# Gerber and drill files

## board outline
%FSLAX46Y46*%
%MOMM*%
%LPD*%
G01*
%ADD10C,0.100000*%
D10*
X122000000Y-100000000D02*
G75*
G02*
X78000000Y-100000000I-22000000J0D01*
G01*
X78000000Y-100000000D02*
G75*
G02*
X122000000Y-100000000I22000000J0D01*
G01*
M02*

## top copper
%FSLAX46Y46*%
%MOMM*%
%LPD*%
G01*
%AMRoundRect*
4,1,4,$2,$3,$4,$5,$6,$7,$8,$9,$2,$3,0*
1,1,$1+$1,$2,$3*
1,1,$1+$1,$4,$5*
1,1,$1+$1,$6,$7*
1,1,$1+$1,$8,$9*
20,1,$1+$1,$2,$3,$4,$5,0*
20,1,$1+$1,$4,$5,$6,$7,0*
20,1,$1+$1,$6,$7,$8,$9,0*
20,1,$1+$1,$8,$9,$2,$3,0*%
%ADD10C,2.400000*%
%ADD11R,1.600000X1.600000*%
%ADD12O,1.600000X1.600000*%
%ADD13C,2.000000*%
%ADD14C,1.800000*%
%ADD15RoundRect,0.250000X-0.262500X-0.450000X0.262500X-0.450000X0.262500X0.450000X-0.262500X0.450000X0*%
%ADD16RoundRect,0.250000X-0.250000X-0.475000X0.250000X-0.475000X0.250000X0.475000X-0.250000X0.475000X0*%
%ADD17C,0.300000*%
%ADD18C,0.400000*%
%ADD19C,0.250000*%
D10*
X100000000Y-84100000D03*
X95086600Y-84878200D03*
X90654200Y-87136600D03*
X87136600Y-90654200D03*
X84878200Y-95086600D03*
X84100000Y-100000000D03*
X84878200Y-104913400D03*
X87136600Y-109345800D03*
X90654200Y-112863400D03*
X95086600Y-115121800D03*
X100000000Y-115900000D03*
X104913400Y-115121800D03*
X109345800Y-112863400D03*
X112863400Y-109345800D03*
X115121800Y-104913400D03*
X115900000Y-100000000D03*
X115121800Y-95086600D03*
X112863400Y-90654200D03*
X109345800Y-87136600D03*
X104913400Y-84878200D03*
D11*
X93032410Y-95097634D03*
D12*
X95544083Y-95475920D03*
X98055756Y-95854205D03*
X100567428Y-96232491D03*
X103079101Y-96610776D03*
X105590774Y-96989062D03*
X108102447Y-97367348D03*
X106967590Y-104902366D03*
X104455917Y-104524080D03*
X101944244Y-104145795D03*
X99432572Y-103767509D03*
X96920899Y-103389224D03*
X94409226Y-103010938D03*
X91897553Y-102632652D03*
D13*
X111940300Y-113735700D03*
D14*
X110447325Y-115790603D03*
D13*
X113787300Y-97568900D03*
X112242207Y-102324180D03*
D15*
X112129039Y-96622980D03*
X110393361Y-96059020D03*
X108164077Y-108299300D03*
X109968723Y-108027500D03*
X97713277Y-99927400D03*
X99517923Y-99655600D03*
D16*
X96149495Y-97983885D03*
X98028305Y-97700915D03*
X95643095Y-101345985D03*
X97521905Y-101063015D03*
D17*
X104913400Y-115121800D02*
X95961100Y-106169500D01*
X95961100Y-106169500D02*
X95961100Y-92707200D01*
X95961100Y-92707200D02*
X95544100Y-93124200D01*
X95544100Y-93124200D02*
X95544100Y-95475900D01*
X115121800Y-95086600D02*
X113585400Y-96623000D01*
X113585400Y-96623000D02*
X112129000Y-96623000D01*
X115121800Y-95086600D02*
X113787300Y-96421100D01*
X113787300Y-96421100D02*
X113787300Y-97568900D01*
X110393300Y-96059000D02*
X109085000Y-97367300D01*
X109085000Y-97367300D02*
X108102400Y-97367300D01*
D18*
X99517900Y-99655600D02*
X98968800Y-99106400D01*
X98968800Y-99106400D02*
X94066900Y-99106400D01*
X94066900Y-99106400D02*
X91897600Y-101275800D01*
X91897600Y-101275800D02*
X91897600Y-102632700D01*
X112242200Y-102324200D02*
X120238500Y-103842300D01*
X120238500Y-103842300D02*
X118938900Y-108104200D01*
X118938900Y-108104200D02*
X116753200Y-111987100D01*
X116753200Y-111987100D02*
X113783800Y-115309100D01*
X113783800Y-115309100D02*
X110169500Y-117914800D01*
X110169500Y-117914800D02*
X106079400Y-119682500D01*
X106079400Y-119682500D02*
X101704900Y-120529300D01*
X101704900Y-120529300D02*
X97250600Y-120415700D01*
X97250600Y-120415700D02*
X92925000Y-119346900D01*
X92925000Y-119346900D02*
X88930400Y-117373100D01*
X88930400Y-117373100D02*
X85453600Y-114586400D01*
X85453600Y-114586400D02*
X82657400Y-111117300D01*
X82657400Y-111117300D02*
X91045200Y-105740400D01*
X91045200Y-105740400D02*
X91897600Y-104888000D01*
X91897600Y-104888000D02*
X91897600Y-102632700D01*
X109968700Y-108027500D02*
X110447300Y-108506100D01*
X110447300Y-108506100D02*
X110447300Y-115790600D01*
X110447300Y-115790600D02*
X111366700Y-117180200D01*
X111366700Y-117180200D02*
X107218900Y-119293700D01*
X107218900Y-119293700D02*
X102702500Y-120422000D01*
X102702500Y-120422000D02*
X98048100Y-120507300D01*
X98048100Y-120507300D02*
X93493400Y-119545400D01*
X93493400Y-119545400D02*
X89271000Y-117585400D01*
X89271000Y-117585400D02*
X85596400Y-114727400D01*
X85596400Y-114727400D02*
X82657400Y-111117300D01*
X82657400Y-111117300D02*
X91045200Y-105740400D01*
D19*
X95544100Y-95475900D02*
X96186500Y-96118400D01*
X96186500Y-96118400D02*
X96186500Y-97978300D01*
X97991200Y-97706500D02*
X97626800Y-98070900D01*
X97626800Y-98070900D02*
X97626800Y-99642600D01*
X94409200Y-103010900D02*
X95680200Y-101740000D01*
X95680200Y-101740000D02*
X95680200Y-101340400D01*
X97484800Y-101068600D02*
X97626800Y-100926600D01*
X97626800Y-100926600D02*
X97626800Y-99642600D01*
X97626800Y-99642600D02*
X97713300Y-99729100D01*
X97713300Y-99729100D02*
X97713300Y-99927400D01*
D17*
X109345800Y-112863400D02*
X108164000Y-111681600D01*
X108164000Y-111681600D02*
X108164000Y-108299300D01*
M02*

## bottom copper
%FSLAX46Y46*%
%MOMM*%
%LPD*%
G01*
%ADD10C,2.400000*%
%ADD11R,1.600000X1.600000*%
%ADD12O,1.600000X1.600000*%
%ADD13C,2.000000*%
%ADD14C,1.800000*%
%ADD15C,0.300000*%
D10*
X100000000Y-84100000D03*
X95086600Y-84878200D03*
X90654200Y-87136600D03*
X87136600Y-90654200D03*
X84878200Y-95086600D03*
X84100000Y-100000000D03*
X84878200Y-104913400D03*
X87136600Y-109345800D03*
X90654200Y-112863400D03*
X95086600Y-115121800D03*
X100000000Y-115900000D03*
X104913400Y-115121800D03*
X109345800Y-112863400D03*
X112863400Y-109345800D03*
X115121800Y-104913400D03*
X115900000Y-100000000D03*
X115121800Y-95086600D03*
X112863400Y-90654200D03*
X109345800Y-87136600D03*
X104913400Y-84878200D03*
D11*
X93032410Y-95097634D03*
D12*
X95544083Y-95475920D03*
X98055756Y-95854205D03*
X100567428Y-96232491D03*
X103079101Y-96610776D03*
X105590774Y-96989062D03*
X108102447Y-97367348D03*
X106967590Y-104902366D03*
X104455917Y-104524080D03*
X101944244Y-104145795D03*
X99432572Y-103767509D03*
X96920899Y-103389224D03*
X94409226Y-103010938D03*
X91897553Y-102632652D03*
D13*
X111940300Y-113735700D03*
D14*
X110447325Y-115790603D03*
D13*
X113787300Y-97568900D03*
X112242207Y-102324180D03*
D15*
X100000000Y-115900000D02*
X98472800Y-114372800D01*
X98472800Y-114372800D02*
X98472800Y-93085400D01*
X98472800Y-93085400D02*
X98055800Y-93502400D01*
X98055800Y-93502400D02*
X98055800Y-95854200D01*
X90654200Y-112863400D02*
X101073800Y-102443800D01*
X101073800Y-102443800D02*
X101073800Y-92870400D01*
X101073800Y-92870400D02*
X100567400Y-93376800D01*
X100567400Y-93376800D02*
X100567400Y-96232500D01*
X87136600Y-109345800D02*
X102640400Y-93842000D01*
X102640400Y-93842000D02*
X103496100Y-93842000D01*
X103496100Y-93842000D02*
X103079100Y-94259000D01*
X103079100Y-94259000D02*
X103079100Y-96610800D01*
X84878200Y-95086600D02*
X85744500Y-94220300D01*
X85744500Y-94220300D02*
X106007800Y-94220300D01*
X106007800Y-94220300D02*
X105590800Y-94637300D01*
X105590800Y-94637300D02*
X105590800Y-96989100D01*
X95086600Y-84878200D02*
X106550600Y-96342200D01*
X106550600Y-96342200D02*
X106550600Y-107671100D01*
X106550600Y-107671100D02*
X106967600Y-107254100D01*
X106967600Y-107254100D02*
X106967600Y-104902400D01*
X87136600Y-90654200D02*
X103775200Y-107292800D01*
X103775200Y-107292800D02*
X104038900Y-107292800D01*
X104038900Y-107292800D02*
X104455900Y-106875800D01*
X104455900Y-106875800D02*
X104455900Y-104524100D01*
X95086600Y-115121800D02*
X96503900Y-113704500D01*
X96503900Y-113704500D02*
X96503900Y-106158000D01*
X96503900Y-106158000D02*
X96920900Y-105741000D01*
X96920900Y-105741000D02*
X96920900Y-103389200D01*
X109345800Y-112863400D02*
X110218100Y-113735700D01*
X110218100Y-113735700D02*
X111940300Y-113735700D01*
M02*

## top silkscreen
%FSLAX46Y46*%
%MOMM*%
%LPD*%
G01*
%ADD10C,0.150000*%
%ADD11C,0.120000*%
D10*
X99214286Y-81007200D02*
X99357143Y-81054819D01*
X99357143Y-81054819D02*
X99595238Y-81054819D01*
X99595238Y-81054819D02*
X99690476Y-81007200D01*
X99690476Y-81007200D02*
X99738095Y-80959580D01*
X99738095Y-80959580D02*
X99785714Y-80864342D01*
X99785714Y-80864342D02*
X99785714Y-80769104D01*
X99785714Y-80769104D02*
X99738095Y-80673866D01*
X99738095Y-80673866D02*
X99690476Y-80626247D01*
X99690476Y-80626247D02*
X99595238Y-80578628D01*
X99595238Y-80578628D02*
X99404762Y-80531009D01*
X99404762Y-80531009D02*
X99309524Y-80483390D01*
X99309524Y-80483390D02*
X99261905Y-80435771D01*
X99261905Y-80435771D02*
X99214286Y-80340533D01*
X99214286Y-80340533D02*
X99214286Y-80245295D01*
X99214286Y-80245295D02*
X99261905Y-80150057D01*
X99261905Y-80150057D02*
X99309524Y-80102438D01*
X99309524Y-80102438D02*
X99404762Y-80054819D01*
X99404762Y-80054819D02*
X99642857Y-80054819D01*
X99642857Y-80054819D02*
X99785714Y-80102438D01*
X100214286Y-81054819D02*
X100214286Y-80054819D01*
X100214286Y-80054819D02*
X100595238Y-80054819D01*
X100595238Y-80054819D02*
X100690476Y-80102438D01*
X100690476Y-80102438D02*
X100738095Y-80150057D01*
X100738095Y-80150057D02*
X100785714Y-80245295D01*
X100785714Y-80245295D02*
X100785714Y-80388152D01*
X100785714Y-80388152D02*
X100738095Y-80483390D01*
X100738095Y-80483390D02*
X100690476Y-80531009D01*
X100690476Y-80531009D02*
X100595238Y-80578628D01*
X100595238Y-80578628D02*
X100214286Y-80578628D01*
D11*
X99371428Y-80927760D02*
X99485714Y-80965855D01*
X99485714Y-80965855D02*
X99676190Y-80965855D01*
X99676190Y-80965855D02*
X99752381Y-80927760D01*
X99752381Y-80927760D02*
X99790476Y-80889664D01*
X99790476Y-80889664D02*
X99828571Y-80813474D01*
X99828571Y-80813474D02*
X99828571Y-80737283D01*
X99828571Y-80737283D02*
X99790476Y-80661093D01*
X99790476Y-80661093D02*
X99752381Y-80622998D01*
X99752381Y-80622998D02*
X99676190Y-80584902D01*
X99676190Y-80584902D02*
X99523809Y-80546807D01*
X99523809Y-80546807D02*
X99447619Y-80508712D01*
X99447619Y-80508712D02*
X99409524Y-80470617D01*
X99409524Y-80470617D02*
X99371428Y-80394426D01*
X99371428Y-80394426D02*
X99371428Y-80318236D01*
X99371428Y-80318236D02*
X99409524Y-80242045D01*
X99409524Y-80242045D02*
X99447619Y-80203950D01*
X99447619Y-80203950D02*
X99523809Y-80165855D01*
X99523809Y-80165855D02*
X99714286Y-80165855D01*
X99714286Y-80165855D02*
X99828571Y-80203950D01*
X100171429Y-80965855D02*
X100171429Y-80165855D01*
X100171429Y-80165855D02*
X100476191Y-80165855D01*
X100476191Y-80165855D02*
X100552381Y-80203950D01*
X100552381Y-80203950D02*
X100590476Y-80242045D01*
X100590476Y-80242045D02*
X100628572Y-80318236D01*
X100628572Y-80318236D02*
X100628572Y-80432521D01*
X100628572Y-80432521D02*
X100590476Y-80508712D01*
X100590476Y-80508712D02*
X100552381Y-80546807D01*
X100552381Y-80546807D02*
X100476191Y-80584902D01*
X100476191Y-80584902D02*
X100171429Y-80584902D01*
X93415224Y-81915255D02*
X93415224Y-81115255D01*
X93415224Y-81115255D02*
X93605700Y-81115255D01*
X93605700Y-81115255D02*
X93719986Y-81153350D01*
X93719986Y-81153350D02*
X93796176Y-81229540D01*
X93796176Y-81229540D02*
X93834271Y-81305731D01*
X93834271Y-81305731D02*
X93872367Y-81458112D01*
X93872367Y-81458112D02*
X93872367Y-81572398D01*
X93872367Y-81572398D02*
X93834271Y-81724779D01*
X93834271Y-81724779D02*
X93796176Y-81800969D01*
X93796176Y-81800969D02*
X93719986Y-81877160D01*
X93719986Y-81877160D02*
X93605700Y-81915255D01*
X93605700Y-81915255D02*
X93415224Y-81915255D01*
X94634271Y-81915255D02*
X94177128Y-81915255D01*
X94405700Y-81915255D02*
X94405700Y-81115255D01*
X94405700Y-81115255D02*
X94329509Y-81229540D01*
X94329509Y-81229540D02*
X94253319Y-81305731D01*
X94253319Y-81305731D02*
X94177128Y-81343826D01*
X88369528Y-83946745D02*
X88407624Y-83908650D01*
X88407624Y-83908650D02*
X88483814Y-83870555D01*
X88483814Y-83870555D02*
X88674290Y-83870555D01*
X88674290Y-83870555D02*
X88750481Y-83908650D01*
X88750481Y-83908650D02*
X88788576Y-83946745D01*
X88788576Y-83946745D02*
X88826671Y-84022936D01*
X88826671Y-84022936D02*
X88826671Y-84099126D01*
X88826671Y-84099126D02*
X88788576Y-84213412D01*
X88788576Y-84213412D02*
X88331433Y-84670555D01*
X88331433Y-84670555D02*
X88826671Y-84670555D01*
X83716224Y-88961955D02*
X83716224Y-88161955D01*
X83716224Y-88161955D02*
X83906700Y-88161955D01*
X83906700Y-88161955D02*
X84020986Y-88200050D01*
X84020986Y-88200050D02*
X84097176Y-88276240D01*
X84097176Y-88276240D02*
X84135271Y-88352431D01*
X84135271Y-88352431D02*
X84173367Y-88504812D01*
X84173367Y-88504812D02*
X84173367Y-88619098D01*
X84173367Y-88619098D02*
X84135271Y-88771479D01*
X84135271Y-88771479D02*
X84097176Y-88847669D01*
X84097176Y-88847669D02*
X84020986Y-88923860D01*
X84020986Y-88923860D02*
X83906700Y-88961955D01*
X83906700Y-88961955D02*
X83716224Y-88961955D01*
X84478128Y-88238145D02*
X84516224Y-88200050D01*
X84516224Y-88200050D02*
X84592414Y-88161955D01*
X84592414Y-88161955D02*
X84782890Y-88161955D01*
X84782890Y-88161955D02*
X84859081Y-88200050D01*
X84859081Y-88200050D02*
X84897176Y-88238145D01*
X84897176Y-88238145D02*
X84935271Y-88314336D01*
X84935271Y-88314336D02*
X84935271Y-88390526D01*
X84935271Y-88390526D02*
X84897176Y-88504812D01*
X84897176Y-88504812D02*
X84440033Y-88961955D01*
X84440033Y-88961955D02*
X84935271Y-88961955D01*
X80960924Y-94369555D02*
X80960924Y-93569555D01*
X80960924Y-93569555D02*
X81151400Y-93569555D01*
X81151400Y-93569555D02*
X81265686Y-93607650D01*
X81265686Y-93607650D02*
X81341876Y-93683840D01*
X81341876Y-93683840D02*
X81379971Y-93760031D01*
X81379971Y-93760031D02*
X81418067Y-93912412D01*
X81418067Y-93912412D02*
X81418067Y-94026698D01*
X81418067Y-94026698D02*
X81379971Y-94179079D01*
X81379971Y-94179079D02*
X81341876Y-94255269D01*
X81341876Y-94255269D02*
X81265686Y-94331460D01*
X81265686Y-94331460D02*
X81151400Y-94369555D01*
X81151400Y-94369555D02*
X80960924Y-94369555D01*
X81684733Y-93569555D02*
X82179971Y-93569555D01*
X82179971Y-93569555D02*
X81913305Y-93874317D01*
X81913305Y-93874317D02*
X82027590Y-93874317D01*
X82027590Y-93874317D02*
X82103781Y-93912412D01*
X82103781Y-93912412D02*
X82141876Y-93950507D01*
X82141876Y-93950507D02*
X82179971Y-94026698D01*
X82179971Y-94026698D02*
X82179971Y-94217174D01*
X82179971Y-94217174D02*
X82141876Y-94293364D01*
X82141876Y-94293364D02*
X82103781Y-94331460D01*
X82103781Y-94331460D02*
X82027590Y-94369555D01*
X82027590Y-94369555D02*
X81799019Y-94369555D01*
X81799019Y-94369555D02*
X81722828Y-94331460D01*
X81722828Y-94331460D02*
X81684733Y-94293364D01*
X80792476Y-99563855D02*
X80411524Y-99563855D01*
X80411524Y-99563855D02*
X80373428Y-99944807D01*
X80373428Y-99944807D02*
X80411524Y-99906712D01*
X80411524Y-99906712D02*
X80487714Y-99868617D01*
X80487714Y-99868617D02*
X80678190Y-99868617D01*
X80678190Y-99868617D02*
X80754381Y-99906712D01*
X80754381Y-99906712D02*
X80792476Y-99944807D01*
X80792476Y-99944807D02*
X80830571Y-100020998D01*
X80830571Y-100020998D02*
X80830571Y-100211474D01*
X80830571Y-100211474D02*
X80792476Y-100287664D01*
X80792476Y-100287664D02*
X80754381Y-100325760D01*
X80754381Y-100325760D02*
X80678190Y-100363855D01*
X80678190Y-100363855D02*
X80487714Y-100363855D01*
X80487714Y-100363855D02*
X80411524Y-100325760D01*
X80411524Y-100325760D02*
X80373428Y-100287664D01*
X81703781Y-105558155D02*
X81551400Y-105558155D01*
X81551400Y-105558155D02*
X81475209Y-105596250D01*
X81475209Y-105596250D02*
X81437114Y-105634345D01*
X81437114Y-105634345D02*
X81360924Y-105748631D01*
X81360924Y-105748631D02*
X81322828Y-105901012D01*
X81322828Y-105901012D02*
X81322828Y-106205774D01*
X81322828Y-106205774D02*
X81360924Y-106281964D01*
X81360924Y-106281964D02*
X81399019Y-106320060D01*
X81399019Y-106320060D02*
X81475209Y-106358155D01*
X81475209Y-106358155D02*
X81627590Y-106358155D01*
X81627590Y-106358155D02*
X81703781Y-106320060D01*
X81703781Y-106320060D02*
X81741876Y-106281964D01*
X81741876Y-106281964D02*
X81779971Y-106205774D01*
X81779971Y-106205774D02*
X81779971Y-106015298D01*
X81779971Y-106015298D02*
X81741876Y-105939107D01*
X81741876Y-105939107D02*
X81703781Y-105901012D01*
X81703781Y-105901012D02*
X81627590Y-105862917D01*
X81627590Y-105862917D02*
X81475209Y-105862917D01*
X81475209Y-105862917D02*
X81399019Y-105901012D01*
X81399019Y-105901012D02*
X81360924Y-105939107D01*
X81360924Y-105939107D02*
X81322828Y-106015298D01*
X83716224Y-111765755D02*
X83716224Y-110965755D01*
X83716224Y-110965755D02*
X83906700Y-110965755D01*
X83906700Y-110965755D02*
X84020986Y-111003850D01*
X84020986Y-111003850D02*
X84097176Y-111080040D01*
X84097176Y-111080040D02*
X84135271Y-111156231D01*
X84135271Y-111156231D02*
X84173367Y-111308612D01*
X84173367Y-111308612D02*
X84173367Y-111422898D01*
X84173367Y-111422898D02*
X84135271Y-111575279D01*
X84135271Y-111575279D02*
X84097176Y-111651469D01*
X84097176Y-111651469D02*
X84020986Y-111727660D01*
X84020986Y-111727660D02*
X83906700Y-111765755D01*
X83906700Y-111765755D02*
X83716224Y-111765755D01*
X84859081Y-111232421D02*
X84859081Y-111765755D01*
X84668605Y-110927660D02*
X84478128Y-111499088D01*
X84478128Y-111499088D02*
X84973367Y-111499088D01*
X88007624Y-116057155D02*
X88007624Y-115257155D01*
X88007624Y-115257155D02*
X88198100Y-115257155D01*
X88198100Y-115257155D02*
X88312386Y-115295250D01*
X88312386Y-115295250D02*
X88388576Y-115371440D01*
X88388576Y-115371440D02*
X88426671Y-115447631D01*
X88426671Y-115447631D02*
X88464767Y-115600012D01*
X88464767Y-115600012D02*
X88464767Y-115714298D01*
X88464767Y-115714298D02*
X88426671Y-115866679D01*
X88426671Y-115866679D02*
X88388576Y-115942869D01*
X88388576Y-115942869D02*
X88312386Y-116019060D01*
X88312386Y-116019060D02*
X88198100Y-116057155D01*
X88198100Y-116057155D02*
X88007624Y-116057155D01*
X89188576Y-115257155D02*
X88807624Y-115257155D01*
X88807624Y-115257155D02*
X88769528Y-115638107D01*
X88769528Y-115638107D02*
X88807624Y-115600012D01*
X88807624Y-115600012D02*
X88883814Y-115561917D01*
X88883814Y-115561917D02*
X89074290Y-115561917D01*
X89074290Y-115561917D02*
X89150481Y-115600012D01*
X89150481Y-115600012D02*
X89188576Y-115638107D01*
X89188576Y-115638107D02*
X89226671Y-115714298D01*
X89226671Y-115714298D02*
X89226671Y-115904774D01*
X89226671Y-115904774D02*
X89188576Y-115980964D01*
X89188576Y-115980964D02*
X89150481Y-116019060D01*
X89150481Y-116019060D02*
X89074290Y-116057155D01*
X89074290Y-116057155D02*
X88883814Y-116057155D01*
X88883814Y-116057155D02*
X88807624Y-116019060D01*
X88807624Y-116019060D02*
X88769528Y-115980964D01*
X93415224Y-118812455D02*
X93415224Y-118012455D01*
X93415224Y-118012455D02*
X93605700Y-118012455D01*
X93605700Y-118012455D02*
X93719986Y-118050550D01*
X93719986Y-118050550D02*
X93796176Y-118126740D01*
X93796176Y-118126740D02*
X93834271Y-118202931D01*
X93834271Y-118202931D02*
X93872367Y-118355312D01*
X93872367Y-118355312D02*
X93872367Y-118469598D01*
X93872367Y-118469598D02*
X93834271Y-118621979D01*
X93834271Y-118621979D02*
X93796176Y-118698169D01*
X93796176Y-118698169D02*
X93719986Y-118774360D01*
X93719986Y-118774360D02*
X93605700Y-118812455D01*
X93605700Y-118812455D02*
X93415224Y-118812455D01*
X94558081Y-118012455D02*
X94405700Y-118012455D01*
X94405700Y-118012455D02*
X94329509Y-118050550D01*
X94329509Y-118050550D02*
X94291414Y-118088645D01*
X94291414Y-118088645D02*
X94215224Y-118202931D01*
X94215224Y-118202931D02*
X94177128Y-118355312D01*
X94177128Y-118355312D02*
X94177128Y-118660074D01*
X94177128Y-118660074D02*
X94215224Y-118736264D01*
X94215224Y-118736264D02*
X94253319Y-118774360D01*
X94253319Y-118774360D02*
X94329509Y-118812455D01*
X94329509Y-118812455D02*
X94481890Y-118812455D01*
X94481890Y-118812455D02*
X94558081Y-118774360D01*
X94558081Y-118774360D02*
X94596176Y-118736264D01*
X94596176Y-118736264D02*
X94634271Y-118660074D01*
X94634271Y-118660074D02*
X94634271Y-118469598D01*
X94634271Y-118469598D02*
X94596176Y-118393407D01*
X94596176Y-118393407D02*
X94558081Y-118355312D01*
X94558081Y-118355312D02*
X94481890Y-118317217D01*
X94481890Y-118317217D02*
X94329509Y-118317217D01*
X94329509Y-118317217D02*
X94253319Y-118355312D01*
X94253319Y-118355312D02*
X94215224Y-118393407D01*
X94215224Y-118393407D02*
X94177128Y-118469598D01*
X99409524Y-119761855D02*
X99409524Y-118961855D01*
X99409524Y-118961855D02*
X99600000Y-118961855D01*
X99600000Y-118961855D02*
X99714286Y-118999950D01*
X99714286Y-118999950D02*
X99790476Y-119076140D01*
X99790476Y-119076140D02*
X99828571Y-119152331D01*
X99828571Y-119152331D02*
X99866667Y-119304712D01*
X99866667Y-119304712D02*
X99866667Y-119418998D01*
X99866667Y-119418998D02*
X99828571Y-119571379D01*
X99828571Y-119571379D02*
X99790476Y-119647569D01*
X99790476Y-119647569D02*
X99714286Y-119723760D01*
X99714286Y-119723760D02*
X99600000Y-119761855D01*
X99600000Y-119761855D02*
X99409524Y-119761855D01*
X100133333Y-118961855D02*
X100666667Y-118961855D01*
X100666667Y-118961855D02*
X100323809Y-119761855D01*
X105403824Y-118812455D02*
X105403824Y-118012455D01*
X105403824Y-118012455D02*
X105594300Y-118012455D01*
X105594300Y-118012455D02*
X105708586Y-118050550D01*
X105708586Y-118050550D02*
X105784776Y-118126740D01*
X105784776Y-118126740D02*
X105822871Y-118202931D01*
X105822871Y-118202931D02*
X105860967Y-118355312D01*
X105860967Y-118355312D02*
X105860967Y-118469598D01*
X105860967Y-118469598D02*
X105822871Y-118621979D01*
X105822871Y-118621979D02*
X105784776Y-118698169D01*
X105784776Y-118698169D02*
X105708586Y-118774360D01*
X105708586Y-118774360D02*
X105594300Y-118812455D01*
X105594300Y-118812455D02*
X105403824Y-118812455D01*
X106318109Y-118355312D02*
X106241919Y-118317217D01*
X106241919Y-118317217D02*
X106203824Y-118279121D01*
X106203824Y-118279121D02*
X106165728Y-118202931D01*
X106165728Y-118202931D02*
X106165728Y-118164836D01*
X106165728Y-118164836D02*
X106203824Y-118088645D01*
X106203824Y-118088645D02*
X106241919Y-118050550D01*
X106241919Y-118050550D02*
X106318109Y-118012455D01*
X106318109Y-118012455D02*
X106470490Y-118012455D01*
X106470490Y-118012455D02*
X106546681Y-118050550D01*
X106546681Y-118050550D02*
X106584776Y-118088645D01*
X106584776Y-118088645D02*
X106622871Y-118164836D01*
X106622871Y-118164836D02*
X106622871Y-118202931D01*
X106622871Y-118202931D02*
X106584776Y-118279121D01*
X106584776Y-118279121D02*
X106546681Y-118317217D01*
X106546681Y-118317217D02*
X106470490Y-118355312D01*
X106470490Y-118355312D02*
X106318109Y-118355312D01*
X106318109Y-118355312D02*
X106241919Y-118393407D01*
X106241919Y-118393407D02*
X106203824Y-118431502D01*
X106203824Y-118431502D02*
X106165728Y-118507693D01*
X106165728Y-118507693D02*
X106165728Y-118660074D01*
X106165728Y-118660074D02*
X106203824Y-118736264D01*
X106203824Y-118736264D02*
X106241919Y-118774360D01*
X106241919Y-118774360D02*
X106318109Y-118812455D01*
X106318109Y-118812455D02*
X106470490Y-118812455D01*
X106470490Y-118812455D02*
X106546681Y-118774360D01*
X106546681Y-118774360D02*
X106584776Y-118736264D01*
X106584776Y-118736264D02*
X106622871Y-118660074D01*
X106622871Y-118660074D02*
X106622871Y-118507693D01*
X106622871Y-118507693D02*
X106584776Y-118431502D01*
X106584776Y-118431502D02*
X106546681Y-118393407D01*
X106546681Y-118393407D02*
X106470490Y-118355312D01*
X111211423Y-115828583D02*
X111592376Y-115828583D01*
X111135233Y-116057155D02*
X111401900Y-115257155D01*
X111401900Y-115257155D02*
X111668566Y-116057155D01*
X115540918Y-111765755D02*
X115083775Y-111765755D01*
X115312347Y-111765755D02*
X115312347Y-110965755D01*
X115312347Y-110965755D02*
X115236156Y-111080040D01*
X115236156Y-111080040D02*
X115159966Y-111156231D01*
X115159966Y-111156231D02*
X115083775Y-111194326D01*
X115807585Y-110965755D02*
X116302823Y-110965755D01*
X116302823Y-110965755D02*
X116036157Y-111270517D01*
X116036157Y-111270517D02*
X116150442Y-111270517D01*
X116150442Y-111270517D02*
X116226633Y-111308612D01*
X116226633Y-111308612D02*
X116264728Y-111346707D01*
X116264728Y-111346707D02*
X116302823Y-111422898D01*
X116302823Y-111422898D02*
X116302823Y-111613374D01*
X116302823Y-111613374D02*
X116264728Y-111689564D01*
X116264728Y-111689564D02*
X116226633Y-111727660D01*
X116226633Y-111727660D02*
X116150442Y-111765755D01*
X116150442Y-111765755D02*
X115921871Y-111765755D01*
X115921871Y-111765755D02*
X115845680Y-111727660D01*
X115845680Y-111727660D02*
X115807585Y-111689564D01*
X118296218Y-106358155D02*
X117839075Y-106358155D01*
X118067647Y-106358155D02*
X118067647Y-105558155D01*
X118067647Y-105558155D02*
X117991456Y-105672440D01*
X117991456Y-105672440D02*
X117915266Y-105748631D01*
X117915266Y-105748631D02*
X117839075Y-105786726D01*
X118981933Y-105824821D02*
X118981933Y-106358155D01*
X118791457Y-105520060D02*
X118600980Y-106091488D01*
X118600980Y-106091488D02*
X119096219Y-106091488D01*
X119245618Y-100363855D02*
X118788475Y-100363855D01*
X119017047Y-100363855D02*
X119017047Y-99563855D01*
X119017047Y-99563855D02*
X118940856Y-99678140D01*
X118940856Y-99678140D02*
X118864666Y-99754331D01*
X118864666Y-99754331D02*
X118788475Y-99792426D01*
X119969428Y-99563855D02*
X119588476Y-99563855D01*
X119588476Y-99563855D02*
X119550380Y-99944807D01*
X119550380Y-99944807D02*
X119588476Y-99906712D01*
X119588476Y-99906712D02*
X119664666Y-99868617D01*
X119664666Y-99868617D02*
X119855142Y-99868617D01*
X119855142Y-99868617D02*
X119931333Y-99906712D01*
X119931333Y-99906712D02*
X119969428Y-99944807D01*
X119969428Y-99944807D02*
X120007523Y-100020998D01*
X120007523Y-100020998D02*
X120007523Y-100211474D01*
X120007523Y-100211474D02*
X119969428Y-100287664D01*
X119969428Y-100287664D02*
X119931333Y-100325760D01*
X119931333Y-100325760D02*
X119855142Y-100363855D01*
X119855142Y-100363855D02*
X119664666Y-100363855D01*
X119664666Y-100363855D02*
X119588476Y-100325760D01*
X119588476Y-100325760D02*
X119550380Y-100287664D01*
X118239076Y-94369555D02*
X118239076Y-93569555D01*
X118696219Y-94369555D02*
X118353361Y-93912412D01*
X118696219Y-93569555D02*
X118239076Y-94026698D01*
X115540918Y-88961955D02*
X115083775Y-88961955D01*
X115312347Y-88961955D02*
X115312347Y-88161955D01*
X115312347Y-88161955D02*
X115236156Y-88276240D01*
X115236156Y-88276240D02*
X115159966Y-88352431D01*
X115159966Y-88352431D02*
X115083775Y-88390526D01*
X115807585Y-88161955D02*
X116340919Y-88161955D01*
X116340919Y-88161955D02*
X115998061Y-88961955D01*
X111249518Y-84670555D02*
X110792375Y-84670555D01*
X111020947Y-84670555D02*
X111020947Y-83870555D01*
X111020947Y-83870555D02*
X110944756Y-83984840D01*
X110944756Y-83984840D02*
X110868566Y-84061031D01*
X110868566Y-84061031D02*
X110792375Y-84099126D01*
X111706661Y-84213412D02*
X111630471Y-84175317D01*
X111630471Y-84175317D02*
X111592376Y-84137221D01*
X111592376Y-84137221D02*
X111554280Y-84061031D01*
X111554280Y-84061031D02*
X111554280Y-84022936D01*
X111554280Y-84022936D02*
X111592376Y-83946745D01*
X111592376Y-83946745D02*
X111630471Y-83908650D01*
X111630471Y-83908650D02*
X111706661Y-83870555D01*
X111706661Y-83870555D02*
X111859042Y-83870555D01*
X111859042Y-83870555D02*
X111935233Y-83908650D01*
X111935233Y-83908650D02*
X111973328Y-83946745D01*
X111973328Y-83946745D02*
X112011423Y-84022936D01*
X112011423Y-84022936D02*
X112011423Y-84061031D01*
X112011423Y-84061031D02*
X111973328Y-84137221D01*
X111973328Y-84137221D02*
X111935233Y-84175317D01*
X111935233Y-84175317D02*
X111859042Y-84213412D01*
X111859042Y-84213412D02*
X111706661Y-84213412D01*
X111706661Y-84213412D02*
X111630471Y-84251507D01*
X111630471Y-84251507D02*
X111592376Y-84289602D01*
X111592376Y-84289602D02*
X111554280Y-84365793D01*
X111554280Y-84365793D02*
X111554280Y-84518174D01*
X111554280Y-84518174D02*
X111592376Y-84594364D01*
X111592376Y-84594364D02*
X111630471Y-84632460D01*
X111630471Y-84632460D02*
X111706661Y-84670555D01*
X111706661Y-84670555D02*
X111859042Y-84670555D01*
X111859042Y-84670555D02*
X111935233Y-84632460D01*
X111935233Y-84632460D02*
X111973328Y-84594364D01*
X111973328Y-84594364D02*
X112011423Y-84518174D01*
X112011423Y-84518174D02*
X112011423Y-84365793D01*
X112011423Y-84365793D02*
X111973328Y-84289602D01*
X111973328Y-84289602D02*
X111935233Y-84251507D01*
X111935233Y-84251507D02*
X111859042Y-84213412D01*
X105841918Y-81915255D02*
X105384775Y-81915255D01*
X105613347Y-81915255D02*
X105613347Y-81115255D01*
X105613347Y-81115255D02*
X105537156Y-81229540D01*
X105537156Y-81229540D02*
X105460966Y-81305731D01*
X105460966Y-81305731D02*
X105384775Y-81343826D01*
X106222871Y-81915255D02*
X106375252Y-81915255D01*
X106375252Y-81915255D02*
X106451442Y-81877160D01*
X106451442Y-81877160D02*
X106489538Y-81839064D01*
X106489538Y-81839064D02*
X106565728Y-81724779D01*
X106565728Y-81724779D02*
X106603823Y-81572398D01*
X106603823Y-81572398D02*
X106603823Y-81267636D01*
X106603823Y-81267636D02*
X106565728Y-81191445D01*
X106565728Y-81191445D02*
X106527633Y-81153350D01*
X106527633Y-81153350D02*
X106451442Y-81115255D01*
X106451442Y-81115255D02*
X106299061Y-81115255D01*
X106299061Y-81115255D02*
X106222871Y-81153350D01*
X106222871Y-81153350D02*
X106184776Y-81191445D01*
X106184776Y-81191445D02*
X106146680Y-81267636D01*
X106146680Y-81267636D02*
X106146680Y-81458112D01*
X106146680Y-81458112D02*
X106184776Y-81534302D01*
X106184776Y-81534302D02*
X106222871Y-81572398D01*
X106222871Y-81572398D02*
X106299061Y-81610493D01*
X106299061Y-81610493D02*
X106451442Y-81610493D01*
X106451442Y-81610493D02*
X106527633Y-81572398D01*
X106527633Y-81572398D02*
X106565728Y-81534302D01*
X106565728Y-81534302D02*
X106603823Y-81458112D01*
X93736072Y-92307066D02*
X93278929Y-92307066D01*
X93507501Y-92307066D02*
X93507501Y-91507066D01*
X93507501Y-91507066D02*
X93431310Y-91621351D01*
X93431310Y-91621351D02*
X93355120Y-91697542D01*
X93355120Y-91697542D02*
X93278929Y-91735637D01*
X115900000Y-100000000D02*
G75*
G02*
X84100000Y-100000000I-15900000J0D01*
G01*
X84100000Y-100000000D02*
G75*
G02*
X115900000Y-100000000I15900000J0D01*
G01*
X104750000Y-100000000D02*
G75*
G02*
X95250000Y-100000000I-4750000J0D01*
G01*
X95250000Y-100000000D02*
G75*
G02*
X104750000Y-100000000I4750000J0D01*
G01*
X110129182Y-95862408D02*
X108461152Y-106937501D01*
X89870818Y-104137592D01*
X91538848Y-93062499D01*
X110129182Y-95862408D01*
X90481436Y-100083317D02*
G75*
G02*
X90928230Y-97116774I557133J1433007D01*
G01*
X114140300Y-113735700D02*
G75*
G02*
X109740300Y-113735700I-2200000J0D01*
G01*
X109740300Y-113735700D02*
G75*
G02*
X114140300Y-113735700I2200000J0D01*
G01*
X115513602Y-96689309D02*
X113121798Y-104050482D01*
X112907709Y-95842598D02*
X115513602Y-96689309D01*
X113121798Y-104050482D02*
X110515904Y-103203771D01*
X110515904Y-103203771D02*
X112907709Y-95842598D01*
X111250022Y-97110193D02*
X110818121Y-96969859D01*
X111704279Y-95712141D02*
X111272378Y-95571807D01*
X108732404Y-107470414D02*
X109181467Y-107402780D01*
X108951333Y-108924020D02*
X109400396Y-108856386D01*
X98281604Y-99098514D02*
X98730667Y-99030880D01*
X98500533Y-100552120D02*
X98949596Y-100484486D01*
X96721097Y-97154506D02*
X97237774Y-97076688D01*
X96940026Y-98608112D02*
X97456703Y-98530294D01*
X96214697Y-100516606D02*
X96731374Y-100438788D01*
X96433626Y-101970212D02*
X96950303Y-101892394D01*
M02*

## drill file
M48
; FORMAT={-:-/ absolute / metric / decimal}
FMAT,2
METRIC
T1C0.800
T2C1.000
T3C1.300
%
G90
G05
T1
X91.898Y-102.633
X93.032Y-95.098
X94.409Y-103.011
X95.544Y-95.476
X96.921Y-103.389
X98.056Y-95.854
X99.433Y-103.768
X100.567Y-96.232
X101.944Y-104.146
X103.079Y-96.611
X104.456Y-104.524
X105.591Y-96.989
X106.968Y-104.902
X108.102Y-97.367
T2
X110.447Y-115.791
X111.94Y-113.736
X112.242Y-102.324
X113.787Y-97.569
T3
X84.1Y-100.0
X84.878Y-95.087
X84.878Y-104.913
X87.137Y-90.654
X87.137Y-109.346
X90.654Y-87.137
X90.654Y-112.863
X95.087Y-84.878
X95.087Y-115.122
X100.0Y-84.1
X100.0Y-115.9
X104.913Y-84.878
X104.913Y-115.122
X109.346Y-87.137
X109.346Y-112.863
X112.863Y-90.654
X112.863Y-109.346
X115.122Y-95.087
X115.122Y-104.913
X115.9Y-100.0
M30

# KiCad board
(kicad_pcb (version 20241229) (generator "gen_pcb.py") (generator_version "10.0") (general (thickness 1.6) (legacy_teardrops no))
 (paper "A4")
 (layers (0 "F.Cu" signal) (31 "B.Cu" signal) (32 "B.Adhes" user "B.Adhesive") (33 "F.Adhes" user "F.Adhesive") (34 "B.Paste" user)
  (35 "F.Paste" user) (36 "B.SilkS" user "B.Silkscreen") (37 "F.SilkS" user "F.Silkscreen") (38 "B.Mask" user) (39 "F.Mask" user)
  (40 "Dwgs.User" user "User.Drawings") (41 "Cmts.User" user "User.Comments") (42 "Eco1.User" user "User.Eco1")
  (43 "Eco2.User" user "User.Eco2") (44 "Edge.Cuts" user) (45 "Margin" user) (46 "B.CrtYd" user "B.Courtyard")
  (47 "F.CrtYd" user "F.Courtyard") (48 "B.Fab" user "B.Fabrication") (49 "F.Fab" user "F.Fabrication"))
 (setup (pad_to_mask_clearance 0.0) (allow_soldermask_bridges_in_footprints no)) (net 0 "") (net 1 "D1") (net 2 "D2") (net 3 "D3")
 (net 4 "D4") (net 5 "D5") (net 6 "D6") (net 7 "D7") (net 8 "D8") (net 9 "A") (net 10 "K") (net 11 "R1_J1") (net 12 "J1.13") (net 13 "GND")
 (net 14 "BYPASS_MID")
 (gr_circle (center 100.0000 100.0000) (end 122.0000 100.0000) (stroke (width 0.1) (type default)) (fill none) (layer "Edge.Cuts"))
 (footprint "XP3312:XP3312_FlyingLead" (layer "F.Cu") (at 100.0000 100.0000 0.0000) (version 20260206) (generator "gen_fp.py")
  (layer "F.Cu")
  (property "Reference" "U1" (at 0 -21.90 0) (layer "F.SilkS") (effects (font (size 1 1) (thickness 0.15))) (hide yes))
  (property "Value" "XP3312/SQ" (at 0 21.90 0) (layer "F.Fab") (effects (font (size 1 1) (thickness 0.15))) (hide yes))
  (fp_circle (center 0 0) (end 15.9000 0) (stroke (width 0.12) (type solid)) (layer "F.SilkS") (fill none))
  (fp_circle (center 0 0) (end 4.7500 0) (stroke (width 0.12) (type solid)) (layer "F.SilkS") (fill none))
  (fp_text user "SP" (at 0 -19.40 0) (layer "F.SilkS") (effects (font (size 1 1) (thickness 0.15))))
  (pad "SP" thru_hole circle (at -0.0000 -15.9000) (size 2.4 2.4) (drill 1.3) (layers "*.Cu" "*.Mask") (remove_unused_layers no))
  (pad "1" thru_hole circle (at -4.9134 -15.1218) (size 2.4 2.4) (drill 1.3) (layers "*.Cu" "*.Mask") (remove_unused_layers no) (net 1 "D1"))
  (pad "2" thru_hole circle (at -9.3458 -12.8634) (size 2.4 2.4) (drill 1.3) (layers "*.Cu" "*.Mask") (remove_unused_layers no))
  (pad "3" thru_hole circle (at -12.8634 -9.3458) (size 2.4 2.4) (drill 1.3) (layers "*.Cu" "*.Mask") (remove_unused_layers no) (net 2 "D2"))
  (pad "4" thru_hole circle (at -15.1218 -4.9134) (size 2.4 2.4) (drill 1.3) (layers "*.Cu" "*.Mask") (remove_unused_layers no) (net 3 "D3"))
  (pad "5" thru_hole circle (at -15.9000 0.0000) (size 2.4 2.4) (drill 1.3) (layers "*.Cu" "*.Mask") (remove_unused_layers no))
  (pad "6" thru_hole circle (at -15.1218 4.9134) (size 2.4 2.4) (drill 1.3) (layers "*.Cu" "*.Mask") (remove_unused_layers no))
  (pad "7" thru_hole circle (at -12.8634 9.3458) (size 2.4 2.4) (drill 1.3) (layers "*.Cu" "*.Mask") (remove_unused_layers no) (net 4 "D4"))
  (pad "8" thru_hole circle (at -9.3458 12.8634) (size 2.4 2.4) (drill 1.3) (layers "*.Cu" "*.Mask") (remove_unused_layers no) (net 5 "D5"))
  (pad "9" thru_hole circle (at -4.9134 15.1218) (size 2.4 2.4) (drill 1.3) (layers "*.Cu" "*.Mask") (remove_unused_layers no) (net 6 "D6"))
  (pad "10" thru_hole circle (at 0.0000 15.9000) (size 2.4 2.4) (drill 1.3) (layers "*.Cu" "*.Mask") (remove_unused_layers no) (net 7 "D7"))
  (pad "11" thru_hole circle (at 4.9134 15.1218) (size 2.4 2.4) (drill 1.3) (layers "*.Cu" "*.Mask") (remove_unused_layers no) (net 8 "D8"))
  (pad "12" thru_hole circle (at 9.3458 12.8634) (size 2.4 2.4) (drill 1.3) (layers "*.Cu" "*.Mask") (remove_unused_layers no) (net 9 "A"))
  (pad "13" thru_hole circle (at 12.8634 9.3458) (size 2.4 2.4) (drill 1.3) (layers "*.Cu" "*.Mask") (remove_unused_layers no))
  (pad "14" thru_hole circle (at 15.1218 4.9134) (size 2.4 2.4) (drill 1.3) (layers "*.Cu" "*.Mask") (remove_unused_layers no))
  (pad "15" thru_hole circle (at 15.9000 0.0000) (size 2.4 2.4) (drill 1.3) (layers "*.Cu" "*.Mask") (remove_unused_layers no))
  (pad "16" thru_hole circle (at 15.1218 -4.9134) (size 2.4 2.4) (drill 1.3) (layers "*.Cu" "*.Mask") (remove_unused_layers no) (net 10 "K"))
  (pad "17" thru_hole circle (at 12.8634 -9.3458) (size 2.4 2.4) (drill 1.3) (layers "*.Cu" "*.Mask") (remove_unused_layers no))
  (pad "18" thru_hole circle (at 9.3458 -12.8634) (size 2.4 2.4) (drill 1.3) (layers "*.Cu" "*.Mask") (remove_unused_layers no))
  (pad "19" thru_hole circle (at 4.9134 -15.1218) (size 2.4 2.4) (drill 1.3) (layers "*.Cu" "*.Mask") (remove_unused_layers no))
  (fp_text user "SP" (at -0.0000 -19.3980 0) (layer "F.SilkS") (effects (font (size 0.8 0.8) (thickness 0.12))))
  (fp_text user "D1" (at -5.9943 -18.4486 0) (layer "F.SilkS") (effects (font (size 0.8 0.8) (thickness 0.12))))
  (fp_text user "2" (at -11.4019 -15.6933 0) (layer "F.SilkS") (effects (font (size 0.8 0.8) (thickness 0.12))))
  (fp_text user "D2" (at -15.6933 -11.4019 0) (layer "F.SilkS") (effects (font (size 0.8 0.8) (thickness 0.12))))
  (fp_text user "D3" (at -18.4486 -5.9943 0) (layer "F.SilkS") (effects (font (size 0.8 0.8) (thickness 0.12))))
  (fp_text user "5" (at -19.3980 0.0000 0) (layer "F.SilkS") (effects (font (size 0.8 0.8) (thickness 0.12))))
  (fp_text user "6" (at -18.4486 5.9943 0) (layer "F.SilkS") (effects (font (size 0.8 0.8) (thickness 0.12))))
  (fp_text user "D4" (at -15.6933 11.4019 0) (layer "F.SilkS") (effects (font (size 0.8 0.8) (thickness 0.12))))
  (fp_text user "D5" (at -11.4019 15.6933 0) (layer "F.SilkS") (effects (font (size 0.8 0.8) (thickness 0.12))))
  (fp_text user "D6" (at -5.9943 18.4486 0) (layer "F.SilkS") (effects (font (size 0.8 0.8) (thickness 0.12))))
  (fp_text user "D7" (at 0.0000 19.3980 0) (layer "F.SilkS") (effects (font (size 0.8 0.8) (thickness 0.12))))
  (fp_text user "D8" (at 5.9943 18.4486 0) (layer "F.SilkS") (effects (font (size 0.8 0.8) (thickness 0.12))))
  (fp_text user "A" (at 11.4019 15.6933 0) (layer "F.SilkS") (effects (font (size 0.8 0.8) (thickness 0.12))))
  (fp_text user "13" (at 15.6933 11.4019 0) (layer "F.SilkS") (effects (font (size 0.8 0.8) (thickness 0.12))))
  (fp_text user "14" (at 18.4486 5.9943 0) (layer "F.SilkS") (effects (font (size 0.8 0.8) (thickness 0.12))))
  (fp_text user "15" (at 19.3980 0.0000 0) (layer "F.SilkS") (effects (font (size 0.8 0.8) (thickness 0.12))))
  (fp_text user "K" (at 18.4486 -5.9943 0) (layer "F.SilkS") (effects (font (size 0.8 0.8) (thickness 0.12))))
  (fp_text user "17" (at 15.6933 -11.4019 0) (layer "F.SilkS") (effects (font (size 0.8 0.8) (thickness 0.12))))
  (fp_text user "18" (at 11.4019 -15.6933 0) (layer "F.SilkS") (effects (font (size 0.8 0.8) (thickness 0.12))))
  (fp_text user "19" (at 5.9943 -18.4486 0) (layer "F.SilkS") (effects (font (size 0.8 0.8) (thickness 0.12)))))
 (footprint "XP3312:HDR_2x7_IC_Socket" (layer "F.Cu") (at 100.0000 100.0000 -98.5650) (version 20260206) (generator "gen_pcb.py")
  (layer "F.Cu")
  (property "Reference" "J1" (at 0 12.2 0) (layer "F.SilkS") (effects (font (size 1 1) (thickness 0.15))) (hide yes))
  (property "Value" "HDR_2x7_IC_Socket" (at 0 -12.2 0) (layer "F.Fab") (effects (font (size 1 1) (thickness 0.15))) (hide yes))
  (fp_rect (start -5.6 9.4) (end 5.6 -9.4) (stroke (width 0.12) (type solid)) (fill none) (layer "F.SilkS"))
  (fp_arc (start -1.5 9.4) (mid 0 10.6) (end 1.5 9.4) (stroke (width 0.12) (type solid)) (layer "F.SilkS"))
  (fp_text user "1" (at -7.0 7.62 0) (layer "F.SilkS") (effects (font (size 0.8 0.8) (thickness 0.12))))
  (pad "1" thru_hole rect (at -3.81 7.62) (size 1.6 1.6) (drill 0.8) (layers "*.Cu" "*.Mask") (remove_unused_layers no))
  (pad "2" thru_hole oval (at -3.81 5.08) (size 1.6 1.6) (drill 0.8) (layers "*.Cu" "*.Mask") (remove_unused_layers no) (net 8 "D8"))
  (pad "3" thru_hole oval (at -3.81 2.54) (size 1.6 1.6) (drill 0.8) (layers "*.Cu" "*.Mask") (remove_unused_layers no) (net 7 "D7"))
  (pad "4" thru_hole oval (at -3.81 0) (size 1.6 1.6) (drill 0.8) (layers "*.Cu" "*.Mask") (remove_unused_layers no) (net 5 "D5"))
  (pad "5" thru_hole oval (at -3.81 -2.54) (size 1.6 1.6) (drill 0.8) (layers "*.Cu" "*.Mask") (remove_unused_layers no) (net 4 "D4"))
  (pad "6" thru_hole oval (at -3.81 -5.08) (size 1.6 1.6) (drill 0.8) (layers "*.Cu" "*.Mask") (remove_unused_layers no) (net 3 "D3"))
  (pad "7" thru_hole oval (at -3.81 -7.62) (size 1.6 1.6) (drill 0.8) (layers "*.Cu" "*.Mask") (remove_unused_layers no) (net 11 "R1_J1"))
  (pad "8" thru_hole oval (at 3.81 -7.62) (size 1.6 1.6) (drill 0.8) (layers "*.Cu" "*.Mask") (remove_unused_layers no) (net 1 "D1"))
  (pad "9" thru_hole oval (at 3.81 -5.08) (size 1.6 1.6) (drill 0.8) (layers "*.Cu" "*.Mask") (remove_unused_layers no) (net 2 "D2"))
  (pad "10" thru_hole oval (at 3.81 -2.54) (size 1.6 1.6) (drill 0.8) (layers "*.Cu" "*.Mask") (remove_unused_layers no))
  (pad "11" thru_hole oval (at 3.81 0) (size 1.6 1.6) (drill 0.8) (layers "*.Cu" "*.Mask") (remove_unused_layers no))
  (pad "12" thru_hole oval (at 3.81 2.54) (size 1.6 1.6) (drill 0.8) (layers "*.Cu" "*.Mask") (remove_unused_layers no) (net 6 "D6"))
  (pad "13" thru_hole oval (at 3.81 5.08) (size 1.6 1.6) (drill 0.8) (layers "*.Cu" "*.Mask") (remove_unused_layers no) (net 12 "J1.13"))
  (pad "14" thru_hole oval (at 3.81 7.62) (size 1.6 1.6) (drill 0.8) (layers "*.Cu" "*.Mask") (remove_unused_layers no) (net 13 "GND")))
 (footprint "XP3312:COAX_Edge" (layer "B.Cu") (at 111.9403 113.7357 144.0000) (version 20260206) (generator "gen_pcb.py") (layer "F.Cu")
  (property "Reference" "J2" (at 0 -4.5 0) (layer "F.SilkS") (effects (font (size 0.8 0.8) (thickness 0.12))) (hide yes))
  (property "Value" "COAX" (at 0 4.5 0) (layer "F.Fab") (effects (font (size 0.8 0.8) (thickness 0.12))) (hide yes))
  (fp_circle (center 0 0) (end 2.2 0) (stroke (width 0.12) (type solid)) (fill none) (layer "F.SilkS"))
  (pad "1" thru_hole circle (at 0 0) (size 2.0 2.0) (drill 1.0) (layers "*.Cu" "*.Mask") (remove_unused_layers no) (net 9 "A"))
  (pad "2" thru_hole circle (at 0 -2.54) (size 1.8 1.8) (drill 1.0) (layers "*.Cu" "*.Mask") (remove_unused_layers no) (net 13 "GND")))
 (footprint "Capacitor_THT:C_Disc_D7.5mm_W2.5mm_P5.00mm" (layer "F.Cu") (at 113.7873 97.5689 251.9999) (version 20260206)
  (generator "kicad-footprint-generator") (layer "F.Cu")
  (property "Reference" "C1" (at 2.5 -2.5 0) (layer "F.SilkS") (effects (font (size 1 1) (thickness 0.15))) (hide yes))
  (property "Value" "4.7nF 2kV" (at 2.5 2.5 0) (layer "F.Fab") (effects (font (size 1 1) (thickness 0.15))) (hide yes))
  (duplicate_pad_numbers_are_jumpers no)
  (fp_line (start -1.37 -1.37) (end 6.37 -1.37) (stroke (width 0.12) (type solid)) (layer "F.SilkS"))
  (fp_line (start -1.37 1.37) (end -1.37 -1.37) (stroke (width 0.12) (type solid)) (layer "F.SilkS"))
  (fp_line (start 6.37 -1.37) (end 6.37 1.37) (stroke (width 0.12) (type solid)) (layer "F.SilkS"))
  (fp_line (start 6.37 1.37) (end -1.37 1.37) (stroke (width 0.12) (type solid)) (layer "F.SilkS"))
  (pad "1" thru_hole circle (at 0 0) (size 2 2) (drill 1) (layers "*.Cu" "*.Mask") (remove_unused_layers no) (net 10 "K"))
  (pad "2" thru_hole circle (at 5 0) (size 2 2) (drill 1) (layers "*.Cu" "*.Mask") (remove_unused_layers no) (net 13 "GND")))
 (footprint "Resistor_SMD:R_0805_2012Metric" (layer "F.Cu") (at 111.2612 96.3410 161.9999) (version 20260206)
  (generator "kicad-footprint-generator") (layer "F.Cu")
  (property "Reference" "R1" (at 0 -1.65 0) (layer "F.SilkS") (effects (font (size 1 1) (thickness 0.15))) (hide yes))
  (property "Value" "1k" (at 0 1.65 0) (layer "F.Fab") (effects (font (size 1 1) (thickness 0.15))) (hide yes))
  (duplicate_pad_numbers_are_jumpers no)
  (fp_line (start -0.227064 -0.735) (end 0.227064 -0.735) (stroke (width 0.12) (type solid)) (layer "F.SilkS"))
  (fp_line (start -0.227064 0.735) (end 0.227064 0.735) (stroke (width 0.12) (type solid)) (layer "F.SilkS"))
  (pad "1" smd roundrect (at -0.9125 0) (size 1.025 1.4) (layers "F.Cu" "F.Mask" "F.Paste") (roundrect_rratio 0.243902) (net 10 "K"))
  (pad "2" smd roundrect (at 0.9125 0) (size 1.025 1.4) (layers "F.Cu" "F.Mask" "F.Paste") (roundrect_rratio 0.243902) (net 11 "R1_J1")))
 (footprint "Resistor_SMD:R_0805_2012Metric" (layer "F.Cu") (at 109.0664 108.1634 8.5650) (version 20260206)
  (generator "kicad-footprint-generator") (layer "F.Cu")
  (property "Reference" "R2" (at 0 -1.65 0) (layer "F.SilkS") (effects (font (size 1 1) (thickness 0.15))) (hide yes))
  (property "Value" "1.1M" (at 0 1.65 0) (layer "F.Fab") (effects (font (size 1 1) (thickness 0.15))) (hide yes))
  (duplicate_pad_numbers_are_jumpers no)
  (fp_line (start -0.227064 -0.735) (end 0.227064 -0.735) (stroke (width 0.12) (type solid)) (layer "F.SilkS"))
  (fp_line (start -0.227064 0.735) (end 0.227064 0.735) (stroke (width 0.12) (type solid)) (layer "F.SilkS"))
  (pad "1" smd roundrect (at -0.9125 0) (size 1.025 1.4) (layers "F.Cu" "F.Mask" "F.Paste") (roundrect_rratio 0.243902) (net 9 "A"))
  (pad "2" smd roundrect (at 0.9125 0) (size 1.025 1.4) (layers "F.Cu" "F.Mask" "F.Paste") (roundrect_rratio 0.243902) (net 13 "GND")))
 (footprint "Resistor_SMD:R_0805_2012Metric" (layer "F.Cu") (at 98.6156 99.7915 8.5650) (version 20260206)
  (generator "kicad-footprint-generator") (layer "F.Cu")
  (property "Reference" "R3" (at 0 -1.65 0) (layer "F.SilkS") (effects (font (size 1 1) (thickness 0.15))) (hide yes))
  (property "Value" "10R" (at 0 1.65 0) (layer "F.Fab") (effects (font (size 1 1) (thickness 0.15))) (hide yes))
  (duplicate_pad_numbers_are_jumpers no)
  (fp_line (start -0.227064 -0.735) (end 0.227064 -0.735) (stroke (width 0.12) (type solid)) (layer "F.SilkS"))
  (fp_line (start -0.227064 0.735) (end 0.227064 0.735) (stroke (width 0.12) (type solid)) (layer "F.SilkS"))
  (pad "1" smd roundrect (at -0.9125 0) (size 1.025 1.4) (layers "F.Cu" "F.Mask" "F.Paste") (roundrect_rratio 0.243902)
   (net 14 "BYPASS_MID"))
  (pad "2" smd roundrect (at 0.9125 0) (size 1.025 1.4) (layers "F.Cu" "F.Mask" "F.Paste") (roundrect_rratio 0.243902) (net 13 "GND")))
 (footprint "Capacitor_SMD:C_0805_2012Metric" (layer "F.Cu") (at 97.0889 97.8424 8.5650) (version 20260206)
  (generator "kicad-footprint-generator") (layer "F.Cu")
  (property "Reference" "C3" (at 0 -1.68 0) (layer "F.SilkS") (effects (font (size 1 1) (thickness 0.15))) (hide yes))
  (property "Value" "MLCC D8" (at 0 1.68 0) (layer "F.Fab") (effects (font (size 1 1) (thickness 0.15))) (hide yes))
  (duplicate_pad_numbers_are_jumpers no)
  (fp_line (start -0.261252 -0.735) (end 0.261252 -0.735) (stroke (width 0.12) (type solid)) (layer "F.SilkS"))
  (fp_line (start -0.261252 0.735) (end 0.261252 0.735) (stroke (width 0.12) (type solid)) (layer "F.SilkS"))
  (pad "1" smd roundrect (at -0.95 0) (size 1 1.45) (layers "F.Cu" "F.Mask" "F.Paste") (roundrect_rratio 0.25) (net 8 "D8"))
  (pad "2" smd roundrect (at 0.95 0) (size 1 1.45) (layers "F.Cu" "F.Mask" "F.Paste") (roundrect_rratio 0.25) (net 14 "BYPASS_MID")))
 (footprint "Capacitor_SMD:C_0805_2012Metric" (layer "F.Cu") (at 96.5825 101.2045 8.5650) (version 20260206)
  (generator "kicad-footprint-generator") (layer "F.Cu")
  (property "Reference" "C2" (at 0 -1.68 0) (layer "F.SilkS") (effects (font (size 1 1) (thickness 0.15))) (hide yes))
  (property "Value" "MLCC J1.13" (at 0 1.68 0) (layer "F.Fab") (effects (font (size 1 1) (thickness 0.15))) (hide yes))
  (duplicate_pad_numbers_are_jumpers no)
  (fp_line (start -0.261252 -0.735) (end 0.261252 -0.735) (stroke (width 0.12) (type solid)) (layer "F.SilkS"))
  (fp_line (start -0.261252 0.735) (end 0.261252 0.735) (stroke (width 0.12) (type solid)) (layer "F.SilkS"))
  (pad "1" smd roundrect (at -0.95 0) (size 1 1.45) (layers "F.Cu" "F.Mask" "F.Paste") (roundrect_rratio 0.25) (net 12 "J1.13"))
  (pad "2" smd roundrect (at 0.95 0) (size 1 1.45) (layers "F.Cu" "F.Mask" "F.Paste") (roundrect_rratio 0.25) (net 14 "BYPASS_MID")))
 (segment (start 100.0000 115.9000) (end 98.4728 114.3728) (width 0.300) (layer "B.Cu") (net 7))
 (segment (start 98.4728 114.3728) (end 98.4728 93.0854) (width 0.300) (layer "B.Cu") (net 7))
 (segment (start 98.4728 93.0854) (end 98.0558 93.5024) (width 0.300) (layer "B.Cu") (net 7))
 (segment (start 98.0558 93.5024) (end 98.0558 95.8542) (width 0.300) (layer "B.Cu") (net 7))
 (segment (start 90.6542 112.8634) (end 101.0738 102.4438) (width 0.300) (layer "B.Cu") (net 5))
 (segment (start 101.0738 102.4438) (end 101.0738 92.8704) (width 0.300) (layer "B.Cu") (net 5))
 (segment (start 101.0738 92.8704) (end 100.5674 93.3768) (width 0.300) (layer "B.Cu") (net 5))
 (segment (start 100.5674 93.3768) (end 100.5674 96.2325) (width 0.300) (layer "B.Cu") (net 5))
 (segment (start 87.1366 109.3458) (end 102.6404 93.8420) (width 0.300) (layer "B.Cu") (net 4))
 (segment (start 102.6404 93.8420) (end 103.4961 93.8420) (width 0.300) (layer "B.Cu") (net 4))
 (segment (start 103.4961 93.8420) (end 103.0791 94.2590) (width 0.300) (layer "B.Cu") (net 4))
 (segment (start 103.0791 94.2590) (end 103.0791 96.6108) (width 0.300) (layer "B.Cu") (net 4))
 (segment (start 84.8782 95.0866) (end 85.7445 94.2203) (width 0.300) (layer "B.Cu") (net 3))
 (segment (start 85.7445 94.2203) (end 106.0078 94.2203) (width 0.300) (layer "B.Cu") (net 3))
 (segment (start 106.0078 94.2203) (end 105.5908 94.6373) (width 0.300) (layer "B.Cu") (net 3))
 (segment (start 105.5908 94.6373) (end 105.5908 96.9891) (width 0.300) (layer "B.Cu") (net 3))
 (segment (start 95.0866 84.8782) (end 106.5506 96.3422) (width 0.300) (layer "B.Cu") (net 1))
 (segment (start 106.5506 96.3422) (end 106.5506 107.6711) (width 0.300) (layer "B.Cu") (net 1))
 (segment (start 106.5506 107.6711) (end 106.9676 107.2541) (width 0.300) (layer "B.Cu") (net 1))
 (segment (start 106.9676 107.2541) (end 106.9676 104.9024) (width 0.300) (layer "B.Cu") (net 1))
 (segment (start 87.1366 90.6542) (end 103.7752 107.2928) (width 0.300) (layer "B.Cu") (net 2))
 (segment (start 103.7752 107.2928) (end 104.0389 107.2928) (width 0.300) (layer "B.Cu") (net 2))
 (segment (start 104.0389 107.2928) (end 104.4559 106.8758) (width 0.300) (layer "B.Cu") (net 2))
 (segment (start 104.4559 106.8758) (end 104.4559 104.5241) (width 0.300) (layer "B.Cu") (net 2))
 (segment (start 95.0866 115.1218) (end 96.5039 113.7045) (width 0.300) (layer "B.Cu") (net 6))
 (segment (start 96.5039 113.7045) (end 96.5039 106.1580) (width 0.300) (layer "B.Cu") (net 6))
 (segment (start 96.5039 106.1580) (end 96.9209 105.7410) (width 0.300) (layer "B.Cu") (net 6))
 (segment (start 96.9209 105.7410) (end 96.9209 103.3892) (width 0.300) (layer "B.Cu") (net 6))
 (segment (start 104.9134 115.1218) (end 95.9611 106.1695) (width 0.300) (layer "F.Cu") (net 8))
 (segment (start 95.9611 106.1695) (end 95.9611 92.7072) (width 0.300) (layer "F.Cu") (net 8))
 (segment (start 95.9611 92.7072) (end 95.5441 93.1242) (width 0.300) (layer "F.Cu") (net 8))
 (segment (start 95.5441 93.1242) (end 95.5441 95.4759) (width 0.300) (layer "F.Cu") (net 8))
 (segment (start 115.1218 95.0866) (end 113.5854 96.6230) (width 0.300) (layer "F.Cu") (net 10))
 (segment (start 113.5854 96.6230) (end 112.1290 96.6230) (width 0.300) (layer "F.Cu") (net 10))
 (segment (start 115.1218 95.0866) (end 113.7873 96.4211) (width 0.300) (layer "F.Cu") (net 10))
 (segment (start 113.7873 96.4211) (end 113.7873 97.5689) (width 0.300) (layer "F.Cu") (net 10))
 (segment (start 110.3933 96.0590) (end 109.0850 97.3673) (width 0.300) (layer "F.Cu") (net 11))
 (segment (start 109.0850 97.3673) (end 108.1024 97.3673) (width 0.300) (layer "F.Cu") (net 11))
 (segment (start 99.5179 99.6556) (end 98.9688 99.1064) (width 0.400) (layer "F.Cu") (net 13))
 (segment (start 98.9688 99.1064) (end 94.0669 99.1064) (width 0.400) (layer "F.Cu") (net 13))
 (segment (start 94.0669 99.1064) (end 91.8976 101.2758) (width 0.400) (layer "F.Cu") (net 13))
 (segment (start 91.8976 101.2758) (end 91.8976 102.6327) (width 0.400) (layer "F.Cu") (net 13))
 (segment (start 112.2422 102.3242) (end 120.2385 103.8423) (width 0.400) (layer "F.Cu") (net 13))
 (segment (start 120.2385 103.8423) (end 118.9389 108.1042) (width 0.400) (layer "F.Cu") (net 13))
 (segment (start 118.9389 108.1042) (end 116.7532 111.9871) (width 0.400) (layer "F.Cu") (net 13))
 (segment (start 116.7532 111.9871) (end 113.7838 115.3091) (width 0.400) (layer "F.Cu") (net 13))
 (segment (start 113.7838 115.3091) (end 110.1695 117.9148) (width 0.400) (layer "F.Cu") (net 13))
 (segment (start 110.1695 117.9148) (end 106.0794 119.6825) (width 0.400) (layer "F.Cu") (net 13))
 (segment (start 106.0794 119.6825) (end 101.7049 120.5293) (width 0.400) (layer "F.Cu") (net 13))
 (segment (start 101.7049 120.5293) (end 97.2506 120.4157) (width 0.400) (layer "F.Cu") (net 13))
 (segment (start 97.2506 120.4157) (end 92.9250 119.3469) (width 0.400) (layer "F.Cu") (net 13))
 (segment (start 92.9250 119.3469) (end 88.9304 117.3731) (width 0.400) (layer "F.Cu") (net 13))
 (segment (start 88.9304 117.3731) (end 85.4536 114.5864) (width 0.400) (layer "F.Cu") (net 13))
 (segment (start 85.4536 114.5864) (end 82.6574 111.1173) (width 0.400) (layer "F.Cu") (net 13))
 (segment (start 82.6574 111.1173) (end 91.0452 105.7404) (width 0.400) (layer "F.Cu") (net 13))
 (segment (start 91.0452 105.7404) (end 91.8976 104.8880) (width 0.400) (layer "F.Cu") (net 13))
 (segment (start 91.8976 104.8880) (end 91.8976 102.6327) (width 0.400) (layer "F.Cu") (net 13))
 (segment (start 109.9687 108.0275) (end 110.4473 108.5061) (width 0.400) (layer "F.Cu") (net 13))
 (segment (start 110.4473 108.5061) (end 110.4473 115.7906) (width 0.400) (layer "F.Cu") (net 13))
 (segment (start 110.4473 115.7906) (end 111.3667 117.1802) (width 0.400) (layer "F.Cu") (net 13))
 (segment (start 111.3667 117.1802) (end 107.2189 119.2937) (width 0.400) (layer "F.Cu") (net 13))
 (segment (start 107.2189 119.2937) (end 102.7025 120.4220) (width 0.400) (layer "F.Cu") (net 13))
 (segment (start 102.7025 120.4220) (end 98.0481 120.5073) (width 0.400) (layer "F.Cu") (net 13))
 (segment (start 98.0481 120.5073) (end 93.4934 119.5454) (width 0.400) (layer "F.Cu") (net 13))
 (segment (start 93.4934 119.5454) (end 89.2710 117.5854) (width 0.400) (layer "F.Cu") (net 13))
 (segment (start 89.2710 117.5854) (end 85.5964 114.7274) (width 0.400) (layer "F.Cu") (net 13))
 (segment (start 85.5964 114.7274) (end 82.6574 111.1173) (width 0.400) (layer "F.Cu") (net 13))
 (segment (start 82.6574 111.1173) (end 91.0452 105.7404) (width 0.400) (layer "F.Cu") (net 13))
 (segment (start 95.5441 95.4759) (end 96.1865 96.1184) (width 0.250) (layer "F.Cu") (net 8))
 (segment (start 96.1865 96.1184) (end 96.1865 97.9783) (width 0.250) (layer "F.Cu") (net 8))
 (segment (start 97.9912 97.7065) (end 97.6268 98.0709) (width 0.250) (layer "F.Cu") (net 14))
 (segment (start 97.6268 98.0709) (end 97.6268 99.6426) (width 0.250) (layer "F.Cu") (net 14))
 (segment (start 94.4092 103.0109) (end 95.6802 101.7400) (width 0.250) (layer "F.Cu") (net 12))
 (segment (start 95.6802 101.7400) (end 95.6802 101.3404) (width 0.250) (layer "F.Cu") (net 12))
 (segment (start 97.4848 101.0686) (end 97.6268 100.9266) (width 0.250) (layer "F.Cu") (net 14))
 (segment (start 97.6268 100.9266) (end 97.6268 99.6426) (width 0.250) (layer "F.Cu") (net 14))
 (segment (start 97.6268 99.6426) (end 97.7133 99.7291) (width 0.250) (layer "F.Cu") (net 14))
 (segment (start 97.7133 99.7291) (end 97.7133 99.9274) (width 0.250) (layer "F.Cu") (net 14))
 (segment (start 109.3458 112.8634) (end 108.1640 111.6816) (width 0.300) (layer "F.Cu") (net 9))
 (segment (start 108.1640 111.6816) (end 108.1640 108.2993) (width 0.300) (layer "F.Cu") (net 9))
 (segment (start 109.3458 112.8634) (end 110.2181 113.7357) (width 0.300) (layer "B.Cu") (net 9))
 (segment (start 110.2181 113.7357) (end 111.9403 113.7357) (width 0.300) (layer "B.Cu") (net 9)))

